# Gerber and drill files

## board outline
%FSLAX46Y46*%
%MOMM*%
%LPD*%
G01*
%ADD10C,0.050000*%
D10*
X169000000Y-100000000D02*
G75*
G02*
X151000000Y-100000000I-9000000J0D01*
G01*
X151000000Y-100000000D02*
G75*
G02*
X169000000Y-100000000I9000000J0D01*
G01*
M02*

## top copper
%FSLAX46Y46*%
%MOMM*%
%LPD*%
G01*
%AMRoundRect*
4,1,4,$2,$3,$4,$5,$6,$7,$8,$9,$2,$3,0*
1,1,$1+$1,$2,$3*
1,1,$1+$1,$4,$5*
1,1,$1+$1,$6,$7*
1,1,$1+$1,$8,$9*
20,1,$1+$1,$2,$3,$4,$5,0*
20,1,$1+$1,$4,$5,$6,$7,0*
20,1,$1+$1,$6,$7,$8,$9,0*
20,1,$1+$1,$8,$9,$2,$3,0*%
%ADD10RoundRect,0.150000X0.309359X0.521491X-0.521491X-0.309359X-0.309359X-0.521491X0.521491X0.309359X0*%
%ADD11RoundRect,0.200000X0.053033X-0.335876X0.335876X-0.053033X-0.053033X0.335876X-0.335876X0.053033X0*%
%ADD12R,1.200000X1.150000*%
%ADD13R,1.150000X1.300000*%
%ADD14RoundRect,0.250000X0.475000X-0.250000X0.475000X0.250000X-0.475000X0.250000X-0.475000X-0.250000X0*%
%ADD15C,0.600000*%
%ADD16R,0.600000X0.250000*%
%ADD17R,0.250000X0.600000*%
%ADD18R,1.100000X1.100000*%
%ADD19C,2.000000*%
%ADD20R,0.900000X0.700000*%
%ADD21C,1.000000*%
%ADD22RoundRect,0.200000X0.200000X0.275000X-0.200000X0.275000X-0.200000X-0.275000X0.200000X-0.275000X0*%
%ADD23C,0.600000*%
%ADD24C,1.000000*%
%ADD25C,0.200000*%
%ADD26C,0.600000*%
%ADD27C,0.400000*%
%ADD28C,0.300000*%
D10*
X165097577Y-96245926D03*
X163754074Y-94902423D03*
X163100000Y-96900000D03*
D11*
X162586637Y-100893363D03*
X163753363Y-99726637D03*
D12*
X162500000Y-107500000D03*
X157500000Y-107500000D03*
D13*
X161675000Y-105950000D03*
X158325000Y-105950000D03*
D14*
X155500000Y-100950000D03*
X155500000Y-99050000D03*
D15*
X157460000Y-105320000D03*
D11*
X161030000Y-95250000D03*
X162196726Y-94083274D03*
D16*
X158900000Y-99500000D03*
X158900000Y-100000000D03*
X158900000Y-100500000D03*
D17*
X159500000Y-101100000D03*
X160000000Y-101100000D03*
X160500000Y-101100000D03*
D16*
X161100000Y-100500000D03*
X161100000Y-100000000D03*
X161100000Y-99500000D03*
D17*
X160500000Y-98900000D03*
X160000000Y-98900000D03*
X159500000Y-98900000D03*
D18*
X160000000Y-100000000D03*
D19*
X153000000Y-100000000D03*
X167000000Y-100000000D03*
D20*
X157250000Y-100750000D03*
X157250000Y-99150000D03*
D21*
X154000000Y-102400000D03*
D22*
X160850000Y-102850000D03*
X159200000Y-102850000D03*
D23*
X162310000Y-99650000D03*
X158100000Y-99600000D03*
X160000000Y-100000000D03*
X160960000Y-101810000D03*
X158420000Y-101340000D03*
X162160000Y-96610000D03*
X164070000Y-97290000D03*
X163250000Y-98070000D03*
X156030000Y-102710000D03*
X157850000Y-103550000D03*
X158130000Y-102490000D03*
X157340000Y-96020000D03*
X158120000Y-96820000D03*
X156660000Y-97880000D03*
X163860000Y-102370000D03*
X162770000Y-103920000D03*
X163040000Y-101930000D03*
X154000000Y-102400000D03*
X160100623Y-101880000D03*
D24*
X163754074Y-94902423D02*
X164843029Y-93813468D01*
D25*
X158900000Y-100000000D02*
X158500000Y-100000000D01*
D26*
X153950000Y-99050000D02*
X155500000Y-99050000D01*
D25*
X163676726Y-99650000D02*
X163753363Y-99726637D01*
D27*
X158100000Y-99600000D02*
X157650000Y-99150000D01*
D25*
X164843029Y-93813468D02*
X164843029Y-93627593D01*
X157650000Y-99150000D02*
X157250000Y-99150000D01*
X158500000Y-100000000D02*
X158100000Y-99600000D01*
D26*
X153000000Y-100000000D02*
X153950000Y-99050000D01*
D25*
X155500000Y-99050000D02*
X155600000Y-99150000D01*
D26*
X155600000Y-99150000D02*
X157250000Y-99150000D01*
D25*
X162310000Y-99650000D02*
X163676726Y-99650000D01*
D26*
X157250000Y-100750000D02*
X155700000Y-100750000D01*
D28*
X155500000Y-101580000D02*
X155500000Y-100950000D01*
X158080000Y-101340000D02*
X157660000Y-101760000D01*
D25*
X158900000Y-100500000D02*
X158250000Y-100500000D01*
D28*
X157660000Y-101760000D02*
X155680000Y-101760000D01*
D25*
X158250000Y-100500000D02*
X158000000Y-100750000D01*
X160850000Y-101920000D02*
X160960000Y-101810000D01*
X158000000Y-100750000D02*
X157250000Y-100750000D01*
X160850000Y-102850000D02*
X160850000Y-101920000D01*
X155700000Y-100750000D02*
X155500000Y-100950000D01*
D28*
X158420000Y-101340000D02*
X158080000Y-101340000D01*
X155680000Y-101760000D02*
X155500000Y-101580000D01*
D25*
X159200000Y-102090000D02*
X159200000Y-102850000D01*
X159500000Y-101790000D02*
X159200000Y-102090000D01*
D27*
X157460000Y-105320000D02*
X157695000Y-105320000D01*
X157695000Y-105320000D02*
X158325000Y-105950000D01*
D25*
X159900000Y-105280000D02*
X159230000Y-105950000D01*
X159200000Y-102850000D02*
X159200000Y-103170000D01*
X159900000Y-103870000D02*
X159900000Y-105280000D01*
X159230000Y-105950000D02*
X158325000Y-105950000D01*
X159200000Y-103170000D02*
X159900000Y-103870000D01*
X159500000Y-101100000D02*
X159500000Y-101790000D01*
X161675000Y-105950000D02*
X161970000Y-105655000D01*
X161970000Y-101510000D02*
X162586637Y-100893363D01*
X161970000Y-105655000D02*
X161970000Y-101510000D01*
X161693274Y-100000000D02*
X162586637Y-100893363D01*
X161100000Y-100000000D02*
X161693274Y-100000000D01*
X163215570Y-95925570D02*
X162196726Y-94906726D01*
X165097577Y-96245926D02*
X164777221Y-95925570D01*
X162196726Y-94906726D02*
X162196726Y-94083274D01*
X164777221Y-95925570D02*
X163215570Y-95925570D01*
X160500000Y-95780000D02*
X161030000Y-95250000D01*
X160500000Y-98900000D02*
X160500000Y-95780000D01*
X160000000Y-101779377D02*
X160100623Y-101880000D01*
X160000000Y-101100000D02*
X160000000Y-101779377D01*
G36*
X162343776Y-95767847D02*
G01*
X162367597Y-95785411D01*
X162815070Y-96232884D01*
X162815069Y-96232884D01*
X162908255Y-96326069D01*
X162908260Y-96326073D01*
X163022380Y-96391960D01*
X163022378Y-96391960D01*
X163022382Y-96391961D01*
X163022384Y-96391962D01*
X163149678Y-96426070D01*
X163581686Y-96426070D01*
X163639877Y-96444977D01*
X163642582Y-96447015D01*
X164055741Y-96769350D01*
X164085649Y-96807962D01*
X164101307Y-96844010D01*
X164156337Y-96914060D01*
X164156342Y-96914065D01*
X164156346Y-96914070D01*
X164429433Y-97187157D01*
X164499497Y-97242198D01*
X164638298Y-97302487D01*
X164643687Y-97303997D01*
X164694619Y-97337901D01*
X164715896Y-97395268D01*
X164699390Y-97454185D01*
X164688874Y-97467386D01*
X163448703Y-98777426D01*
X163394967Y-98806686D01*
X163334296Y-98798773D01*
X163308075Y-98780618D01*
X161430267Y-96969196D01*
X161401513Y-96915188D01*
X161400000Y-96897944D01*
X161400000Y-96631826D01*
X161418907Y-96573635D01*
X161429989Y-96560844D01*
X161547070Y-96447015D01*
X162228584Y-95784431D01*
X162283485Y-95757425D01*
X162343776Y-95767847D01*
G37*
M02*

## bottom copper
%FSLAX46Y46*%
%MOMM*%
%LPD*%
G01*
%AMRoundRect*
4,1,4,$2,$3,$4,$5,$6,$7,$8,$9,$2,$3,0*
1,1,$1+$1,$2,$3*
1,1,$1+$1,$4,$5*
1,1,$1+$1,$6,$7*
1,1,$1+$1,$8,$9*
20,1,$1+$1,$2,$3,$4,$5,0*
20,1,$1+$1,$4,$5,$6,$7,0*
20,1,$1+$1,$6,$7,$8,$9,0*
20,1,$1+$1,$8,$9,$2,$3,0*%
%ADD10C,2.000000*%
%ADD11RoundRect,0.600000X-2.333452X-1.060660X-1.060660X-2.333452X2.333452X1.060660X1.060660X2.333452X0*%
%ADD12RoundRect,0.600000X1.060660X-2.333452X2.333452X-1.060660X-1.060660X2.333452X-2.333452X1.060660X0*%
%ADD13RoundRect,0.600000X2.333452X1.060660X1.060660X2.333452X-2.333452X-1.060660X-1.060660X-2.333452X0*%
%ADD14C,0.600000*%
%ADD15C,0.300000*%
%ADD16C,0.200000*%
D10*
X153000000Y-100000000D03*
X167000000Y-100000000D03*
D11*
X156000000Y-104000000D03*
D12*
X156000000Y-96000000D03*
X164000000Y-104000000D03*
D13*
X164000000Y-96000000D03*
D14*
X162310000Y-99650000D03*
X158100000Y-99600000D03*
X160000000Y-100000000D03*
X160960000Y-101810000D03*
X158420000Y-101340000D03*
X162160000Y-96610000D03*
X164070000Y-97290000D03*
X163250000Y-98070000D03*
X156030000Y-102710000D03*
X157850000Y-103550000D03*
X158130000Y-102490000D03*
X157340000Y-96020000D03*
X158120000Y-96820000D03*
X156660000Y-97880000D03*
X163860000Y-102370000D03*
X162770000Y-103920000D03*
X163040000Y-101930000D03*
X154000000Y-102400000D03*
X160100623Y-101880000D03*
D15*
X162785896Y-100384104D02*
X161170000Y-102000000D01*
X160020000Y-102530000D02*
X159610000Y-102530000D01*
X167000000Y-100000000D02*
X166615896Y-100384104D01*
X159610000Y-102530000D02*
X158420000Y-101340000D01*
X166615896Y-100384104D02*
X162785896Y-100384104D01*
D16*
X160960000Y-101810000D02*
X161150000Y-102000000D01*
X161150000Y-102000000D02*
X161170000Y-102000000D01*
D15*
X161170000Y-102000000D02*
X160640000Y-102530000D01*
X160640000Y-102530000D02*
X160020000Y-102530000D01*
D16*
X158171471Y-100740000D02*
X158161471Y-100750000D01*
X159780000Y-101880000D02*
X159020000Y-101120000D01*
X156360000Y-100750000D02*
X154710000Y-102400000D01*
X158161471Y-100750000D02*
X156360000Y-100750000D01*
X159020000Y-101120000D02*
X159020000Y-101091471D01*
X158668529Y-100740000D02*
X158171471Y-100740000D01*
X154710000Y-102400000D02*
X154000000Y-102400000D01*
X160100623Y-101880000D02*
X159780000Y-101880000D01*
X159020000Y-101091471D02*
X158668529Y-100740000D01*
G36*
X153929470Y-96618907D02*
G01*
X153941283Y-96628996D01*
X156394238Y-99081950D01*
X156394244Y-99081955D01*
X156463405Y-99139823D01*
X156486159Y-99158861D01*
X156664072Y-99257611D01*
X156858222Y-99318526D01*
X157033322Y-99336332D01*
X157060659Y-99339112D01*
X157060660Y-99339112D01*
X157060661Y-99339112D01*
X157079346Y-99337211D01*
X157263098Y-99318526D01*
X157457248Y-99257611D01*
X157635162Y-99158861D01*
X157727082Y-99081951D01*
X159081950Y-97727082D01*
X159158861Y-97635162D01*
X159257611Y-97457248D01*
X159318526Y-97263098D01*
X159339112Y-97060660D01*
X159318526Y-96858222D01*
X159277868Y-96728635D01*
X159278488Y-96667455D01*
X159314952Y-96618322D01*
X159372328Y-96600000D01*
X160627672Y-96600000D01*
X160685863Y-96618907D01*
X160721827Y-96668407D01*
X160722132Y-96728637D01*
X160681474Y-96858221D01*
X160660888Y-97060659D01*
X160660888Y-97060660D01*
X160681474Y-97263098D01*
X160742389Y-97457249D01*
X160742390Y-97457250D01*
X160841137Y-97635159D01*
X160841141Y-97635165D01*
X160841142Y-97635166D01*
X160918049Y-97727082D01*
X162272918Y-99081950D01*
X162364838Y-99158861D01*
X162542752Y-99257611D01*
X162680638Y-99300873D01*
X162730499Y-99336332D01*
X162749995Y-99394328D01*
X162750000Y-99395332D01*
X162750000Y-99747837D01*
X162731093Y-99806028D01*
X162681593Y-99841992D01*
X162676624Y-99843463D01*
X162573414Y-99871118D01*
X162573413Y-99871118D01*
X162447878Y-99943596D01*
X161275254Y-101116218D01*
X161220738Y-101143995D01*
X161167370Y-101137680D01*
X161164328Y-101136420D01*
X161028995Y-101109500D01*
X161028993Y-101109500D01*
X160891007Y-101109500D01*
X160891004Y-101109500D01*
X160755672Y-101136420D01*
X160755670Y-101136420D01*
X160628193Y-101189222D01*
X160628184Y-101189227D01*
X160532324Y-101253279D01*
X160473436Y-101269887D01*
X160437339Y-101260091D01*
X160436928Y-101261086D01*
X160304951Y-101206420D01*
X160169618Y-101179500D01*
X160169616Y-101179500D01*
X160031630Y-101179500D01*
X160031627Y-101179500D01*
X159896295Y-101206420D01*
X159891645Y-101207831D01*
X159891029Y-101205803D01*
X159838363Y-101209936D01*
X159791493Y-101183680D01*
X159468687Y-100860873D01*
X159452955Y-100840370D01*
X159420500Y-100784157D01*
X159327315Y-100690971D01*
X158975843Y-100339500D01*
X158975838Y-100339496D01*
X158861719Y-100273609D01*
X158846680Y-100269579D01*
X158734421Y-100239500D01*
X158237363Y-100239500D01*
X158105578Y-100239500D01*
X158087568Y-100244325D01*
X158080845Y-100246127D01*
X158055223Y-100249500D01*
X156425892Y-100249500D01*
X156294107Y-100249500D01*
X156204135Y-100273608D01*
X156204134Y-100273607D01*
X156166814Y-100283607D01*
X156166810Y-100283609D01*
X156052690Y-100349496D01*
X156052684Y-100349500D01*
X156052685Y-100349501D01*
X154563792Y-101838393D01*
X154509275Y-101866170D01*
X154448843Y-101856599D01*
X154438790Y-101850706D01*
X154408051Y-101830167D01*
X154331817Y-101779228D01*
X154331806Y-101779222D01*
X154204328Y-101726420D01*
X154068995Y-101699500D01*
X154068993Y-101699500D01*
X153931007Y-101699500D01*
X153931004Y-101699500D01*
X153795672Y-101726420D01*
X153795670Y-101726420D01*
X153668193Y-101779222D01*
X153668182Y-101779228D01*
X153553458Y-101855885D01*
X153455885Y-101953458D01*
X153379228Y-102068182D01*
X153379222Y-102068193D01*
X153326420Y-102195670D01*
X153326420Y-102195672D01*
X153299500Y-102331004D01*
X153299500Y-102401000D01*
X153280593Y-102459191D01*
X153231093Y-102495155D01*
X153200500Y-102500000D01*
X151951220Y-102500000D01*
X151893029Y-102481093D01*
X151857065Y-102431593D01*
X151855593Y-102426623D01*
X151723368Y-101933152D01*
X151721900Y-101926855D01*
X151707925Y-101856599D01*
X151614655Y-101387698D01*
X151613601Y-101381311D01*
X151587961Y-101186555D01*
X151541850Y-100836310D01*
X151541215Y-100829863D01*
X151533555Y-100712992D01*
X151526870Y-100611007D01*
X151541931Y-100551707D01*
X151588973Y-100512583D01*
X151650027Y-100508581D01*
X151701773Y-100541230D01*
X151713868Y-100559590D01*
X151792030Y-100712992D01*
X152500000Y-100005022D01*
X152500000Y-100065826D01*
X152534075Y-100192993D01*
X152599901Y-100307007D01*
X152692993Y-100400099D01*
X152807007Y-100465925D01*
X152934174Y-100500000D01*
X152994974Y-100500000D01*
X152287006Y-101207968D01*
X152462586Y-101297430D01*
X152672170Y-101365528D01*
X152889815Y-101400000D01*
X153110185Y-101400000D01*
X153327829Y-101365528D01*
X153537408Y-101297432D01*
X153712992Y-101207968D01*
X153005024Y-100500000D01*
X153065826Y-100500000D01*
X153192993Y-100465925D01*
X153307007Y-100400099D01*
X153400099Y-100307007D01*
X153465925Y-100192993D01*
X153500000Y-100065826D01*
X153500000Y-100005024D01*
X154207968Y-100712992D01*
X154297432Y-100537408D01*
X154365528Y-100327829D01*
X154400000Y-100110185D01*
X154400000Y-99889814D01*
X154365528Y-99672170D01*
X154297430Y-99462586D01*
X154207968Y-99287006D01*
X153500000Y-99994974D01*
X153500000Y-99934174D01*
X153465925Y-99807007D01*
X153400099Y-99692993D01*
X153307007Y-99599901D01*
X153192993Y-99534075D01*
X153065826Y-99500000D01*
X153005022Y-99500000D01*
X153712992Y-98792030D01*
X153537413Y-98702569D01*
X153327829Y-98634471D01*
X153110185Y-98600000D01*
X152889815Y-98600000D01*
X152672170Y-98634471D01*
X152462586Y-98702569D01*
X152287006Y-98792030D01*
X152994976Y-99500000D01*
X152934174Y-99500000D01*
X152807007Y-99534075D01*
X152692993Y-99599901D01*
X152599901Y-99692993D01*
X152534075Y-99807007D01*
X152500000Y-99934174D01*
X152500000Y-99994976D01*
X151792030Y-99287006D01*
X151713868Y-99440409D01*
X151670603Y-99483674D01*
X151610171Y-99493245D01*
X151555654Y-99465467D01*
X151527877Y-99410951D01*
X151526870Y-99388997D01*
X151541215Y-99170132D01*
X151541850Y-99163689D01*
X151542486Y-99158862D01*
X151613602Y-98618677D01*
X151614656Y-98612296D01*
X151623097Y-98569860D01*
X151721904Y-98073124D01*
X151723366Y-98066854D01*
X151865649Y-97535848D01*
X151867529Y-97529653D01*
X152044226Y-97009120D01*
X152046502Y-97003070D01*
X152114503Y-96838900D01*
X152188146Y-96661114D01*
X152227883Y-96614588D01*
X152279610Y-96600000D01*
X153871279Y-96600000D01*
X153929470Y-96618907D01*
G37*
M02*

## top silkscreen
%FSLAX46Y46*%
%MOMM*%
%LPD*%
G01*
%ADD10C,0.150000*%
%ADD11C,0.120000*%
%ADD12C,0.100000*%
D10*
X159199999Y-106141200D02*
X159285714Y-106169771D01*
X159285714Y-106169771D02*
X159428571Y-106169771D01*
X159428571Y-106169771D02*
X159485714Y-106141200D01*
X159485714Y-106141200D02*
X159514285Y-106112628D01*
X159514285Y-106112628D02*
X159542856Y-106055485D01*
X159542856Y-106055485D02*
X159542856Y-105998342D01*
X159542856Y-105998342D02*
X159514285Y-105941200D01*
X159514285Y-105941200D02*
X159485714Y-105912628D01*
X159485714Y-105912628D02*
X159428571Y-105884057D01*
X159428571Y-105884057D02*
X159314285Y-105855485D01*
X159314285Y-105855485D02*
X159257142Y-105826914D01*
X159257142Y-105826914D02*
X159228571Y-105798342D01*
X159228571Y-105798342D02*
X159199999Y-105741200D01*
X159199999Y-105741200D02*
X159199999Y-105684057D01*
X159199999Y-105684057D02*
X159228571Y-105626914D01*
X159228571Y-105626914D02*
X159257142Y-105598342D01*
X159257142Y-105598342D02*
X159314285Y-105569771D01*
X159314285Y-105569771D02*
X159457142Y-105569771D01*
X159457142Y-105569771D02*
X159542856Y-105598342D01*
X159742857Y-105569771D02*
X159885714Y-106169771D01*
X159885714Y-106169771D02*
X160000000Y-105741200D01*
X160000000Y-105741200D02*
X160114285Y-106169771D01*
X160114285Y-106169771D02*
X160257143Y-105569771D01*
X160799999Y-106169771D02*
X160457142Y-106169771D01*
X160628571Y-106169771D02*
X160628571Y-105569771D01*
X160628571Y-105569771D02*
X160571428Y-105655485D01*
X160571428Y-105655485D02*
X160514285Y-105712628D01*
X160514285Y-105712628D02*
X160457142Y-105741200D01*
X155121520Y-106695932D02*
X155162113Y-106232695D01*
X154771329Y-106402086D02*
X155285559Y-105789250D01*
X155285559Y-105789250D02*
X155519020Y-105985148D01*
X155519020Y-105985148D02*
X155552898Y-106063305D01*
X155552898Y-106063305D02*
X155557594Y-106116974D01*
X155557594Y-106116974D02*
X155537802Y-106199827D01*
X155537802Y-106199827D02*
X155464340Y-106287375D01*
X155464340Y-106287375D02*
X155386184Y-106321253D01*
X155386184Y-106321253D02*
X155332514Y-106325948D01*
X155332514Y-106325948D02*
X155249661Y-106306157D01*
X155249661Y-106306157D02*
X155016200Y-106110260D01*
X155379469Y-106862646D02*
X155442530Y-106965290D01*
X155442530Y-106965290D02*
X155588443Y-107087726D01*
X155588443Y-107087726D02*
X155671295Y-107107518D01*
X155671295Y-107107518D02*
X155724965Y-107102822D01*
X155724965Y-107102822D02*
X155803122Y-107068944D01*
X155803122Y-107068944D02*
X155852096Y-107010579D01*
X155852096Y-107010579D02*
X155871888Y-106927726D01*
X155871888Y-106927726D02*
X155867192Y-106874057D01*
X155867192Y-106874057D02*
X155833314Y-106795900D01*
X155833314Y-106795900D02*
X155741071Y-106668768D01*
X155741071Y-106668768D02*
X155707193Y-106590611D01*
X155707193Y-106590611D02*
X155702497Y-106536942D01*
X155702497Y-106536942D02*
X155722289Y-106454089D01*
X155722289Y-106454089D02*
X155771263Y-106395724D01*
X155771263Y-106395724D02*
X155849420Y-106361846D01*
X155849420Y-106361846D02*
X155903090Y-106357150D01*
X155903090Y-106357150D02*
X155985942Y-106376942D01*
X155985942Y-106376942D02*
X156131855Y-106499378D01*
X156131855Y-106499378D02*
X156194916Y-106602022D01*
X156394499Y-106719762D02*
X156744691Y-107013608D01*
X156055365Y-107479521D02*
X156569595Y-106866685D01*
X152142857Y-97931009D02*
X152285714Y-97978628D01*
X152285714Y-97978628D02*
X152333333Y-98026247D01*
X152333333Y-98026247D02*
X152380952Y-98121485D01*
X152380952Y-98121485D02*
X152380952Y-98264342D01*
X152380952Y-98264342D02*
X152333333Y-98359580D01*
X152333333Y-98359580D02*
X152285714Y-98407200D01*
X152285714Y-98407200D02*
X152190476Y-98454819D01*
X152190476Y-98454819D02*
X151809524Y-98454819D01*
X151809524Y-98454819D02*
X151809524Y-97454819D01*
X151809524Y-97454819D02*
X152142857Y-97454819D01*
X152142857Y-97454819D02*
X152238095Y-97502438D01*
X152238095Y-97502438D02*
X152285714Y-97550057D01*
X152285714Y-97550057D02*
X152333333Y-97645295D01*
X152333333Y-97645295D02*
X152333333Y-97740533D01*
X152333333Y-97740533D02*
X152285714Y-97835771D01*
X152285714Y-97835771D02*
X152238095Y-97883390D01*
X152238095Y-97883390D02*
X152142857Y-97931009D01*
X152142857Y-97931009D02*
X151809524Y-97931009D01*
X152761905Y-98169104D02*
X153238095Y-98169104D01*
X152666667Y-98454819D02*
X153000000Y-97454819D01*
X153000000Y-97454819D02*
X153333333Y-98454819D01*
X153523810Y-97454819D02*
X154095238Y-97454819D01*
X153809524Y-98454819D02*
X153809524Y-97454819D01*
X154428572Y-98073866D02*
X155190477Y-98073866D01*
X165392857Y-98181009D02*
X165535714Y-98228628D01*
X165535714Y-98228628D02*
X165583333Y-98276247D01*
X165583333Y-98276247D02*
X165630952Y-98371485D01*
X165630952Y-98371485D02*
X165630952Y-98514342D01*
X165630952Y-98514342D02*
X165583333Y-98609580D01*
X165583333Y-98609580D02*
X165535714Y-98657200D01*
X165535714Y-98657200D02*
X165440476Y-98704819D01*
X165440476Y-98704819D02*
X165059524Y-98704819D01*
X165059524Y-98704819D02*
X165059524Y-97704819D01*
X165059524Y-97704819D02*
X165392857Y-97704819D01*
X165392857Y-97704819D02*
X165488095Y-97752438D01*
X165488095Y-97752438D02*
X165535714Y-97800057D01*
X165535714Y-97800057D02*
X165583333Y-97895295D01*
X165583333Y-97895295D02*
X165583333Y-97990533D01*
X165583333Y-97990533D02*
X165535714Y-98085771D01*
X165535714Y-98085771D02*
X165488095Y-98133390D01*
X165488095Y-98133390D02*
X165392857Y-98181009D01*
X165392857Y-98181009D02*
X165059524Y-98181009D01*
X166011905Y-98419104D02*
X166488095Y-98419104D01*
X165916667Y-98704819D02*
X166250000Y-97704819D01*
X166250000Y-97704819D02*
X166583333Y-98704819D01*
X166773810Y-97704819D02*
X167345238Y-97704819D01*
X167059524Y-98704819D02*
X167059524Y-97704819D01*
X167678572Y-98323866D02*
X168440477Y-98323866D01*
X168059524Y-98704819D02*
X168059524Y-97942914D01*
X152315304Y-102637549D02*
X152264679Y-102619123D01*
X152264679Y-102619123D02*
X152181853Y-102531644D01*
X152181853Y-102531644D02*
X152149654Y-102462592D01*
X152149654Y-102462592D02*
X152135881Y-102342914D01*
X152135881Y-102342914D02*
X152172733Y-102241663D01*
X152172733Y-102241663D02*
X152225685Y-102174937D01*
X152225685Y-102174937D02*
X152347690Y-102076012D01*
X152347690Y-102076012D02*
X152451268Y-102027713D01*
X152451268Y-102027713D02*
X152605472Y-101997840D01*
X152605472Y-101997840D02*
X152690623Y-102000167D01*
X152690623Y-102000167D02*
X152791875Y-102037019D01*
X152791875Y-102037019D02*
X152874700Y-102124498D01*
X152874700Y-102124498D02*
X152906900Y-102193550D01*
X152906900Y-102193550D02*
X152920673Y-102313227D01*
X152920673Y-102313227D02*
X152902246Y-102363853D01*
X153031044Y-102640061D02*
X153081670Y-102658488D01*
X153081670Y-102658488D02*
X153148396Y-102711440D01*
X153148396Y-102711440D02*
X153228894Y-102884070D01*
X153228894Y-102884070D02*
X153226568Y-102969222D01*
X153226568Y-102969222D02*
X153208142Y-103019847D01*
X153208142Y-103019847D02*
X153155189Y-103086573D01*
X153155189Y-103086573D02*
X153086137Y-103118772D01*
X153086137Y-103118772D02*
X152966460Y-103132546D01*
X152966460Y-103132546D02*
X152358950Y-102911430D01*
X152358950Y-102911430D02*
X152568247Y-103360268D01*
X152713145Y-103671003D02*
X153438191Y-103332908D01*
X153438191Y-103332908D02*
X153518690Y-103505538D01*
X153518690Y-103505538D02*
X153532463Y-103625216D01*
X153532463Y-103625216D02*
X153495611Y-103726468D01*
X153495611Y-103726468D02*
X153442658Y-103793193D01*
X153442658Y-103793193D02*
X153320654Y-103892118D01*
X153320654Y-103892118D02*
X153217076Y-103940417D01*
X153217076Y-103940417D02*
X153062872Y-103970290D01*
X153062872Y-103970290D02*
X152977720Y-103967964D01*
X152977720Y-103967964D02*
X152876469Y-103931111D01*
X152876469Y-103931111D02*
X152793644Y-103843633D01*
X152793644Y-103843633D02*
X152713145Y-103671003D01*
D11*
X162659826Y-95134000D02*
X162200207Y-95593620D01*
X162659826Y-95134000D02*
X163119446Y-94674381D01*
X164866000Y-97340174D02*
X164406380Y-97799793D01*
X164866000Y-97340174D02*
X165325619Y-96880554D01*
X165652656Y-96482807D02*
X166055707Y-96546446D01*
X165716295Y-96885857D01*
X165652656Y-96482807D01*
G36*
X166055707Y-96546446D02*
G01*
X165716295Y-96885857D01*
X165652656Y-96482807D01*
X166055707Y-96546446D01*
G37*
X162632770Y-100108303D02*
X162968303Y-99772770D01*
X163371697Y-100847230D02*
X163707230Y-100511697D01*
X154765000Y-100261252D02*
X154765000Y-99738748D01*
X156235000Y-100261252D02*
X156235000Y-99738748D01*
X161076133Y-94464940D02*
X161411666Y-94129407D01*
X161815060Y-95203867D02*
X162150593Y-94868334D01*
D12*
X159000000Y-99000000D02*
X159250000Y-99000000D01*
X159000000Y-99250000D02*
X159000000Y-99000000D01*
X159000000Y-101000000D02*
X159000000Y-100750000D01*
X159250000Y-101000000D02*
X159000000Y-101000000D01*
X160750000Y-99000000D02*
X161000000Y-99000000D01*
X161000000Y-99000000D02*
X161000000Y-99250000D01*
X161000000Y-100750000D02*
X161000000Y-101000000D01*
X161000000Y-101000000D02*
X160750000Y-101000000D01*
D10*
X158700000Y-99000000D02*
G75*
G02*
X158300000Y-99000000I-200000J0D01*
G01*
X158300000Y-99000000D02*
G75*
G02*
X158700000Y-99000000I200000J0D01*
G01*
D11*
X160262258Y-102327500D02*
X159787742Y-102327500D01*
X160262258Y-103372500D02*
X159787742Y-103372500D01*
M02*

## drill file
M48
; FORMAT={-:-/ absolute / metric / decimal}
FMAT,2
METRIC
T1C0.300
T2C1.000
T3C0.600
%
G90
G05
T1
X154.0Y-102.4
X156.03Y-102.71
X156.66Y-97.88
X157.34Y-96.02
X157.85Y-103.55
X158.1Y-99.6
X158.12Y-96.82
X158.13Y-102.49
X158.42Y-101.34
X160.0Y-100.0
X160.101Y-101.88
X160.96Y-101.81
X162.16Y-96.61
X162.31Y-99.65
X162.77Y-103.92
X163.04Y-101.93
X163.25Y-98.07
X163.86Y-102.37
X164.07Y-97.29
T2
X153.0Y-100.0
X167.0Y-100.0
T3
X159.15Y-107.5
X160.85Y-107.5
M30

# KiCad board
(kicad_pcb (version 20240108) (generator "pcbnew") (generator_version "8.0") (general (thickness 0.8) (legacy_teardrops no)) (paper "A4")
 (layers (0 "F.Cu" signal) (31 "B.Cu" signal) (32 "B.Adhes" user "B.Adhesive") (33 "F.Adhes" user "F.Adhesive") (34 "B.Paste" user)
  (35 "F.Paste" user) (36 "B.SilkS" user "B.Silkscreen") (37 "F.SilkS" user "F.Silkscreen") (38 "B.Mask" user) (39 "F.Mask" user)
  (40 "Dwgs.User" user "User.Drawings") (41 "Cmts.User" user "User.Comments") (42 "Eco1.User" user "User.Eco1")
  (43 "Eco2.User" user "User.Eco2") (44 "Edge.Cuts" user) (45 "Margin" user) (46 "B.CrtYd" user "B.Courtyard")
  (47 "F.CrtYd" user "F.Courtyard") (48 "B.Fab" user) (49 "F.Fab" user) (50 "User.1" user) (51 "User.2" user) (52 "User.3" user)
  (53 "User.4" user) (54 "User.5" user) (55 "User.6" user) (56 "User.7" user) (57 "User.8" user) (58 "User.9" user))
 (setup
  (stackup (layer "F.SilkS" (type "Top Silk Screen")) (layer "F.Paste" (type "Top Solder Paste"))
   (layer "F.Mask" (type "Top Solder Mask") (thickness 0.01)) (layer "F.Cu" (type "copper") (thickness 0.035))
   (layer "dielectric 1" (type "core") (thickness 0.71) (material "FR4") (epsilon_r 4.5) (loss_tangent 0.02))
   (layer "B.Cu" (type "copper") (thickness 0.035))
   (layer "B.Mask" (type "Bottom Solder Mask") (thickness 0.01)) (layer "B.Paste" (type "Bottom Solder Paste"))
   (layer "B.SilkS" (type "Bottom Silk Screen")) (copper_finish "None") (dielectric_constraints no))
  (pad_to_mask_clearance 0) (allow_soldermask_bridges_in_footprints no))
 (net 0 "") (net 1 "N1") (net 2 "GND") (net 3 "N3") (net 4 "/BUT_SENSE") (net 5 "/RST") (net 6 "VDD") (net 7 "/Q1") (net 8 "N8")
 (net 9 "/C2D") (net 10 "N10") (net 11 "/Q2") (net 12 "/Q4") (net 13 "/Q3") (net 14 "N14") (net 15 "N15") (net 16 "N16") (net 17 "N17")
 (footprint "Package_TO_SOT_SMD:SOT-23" (layer "F.Cu") (at 163.762913 96.237087 -135)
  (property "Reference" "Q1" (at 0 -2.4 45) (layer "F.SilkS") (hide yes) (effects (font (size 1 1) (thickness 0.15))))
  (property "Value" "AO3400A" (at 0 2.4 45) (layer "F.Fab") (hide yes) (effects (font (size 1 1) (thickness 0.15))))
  (fp_line (start 0 1.560001) (end 0.65 1.56) (stroke (width 0.12) (type solid)) (layer "F.SilkS"))
  (fp_line (start 0 1.560001) (end -0.65 1.56) (stroke (width 0.12) (type solid)) (layer "F.SilkS"))
  (fp_line (start 0 -1.560001) (end 0.65 -1.56) (stroke (width 0.12) (type solid)) (layer "F.SilkS"))
  (fp_line (start 0 -1.560001) (end -0.65 -1.56) (stroke (width 0.12) (type solid)) (layer "F.SilkS"))
  (fp_poly
   (pts (xy -1.1625 -1.51) (xy -1.4025 -1.84) (xy -0.9225 -1.839999) (xy -1.1625 -1.51)) (stroke (width 0.12) (type solid)) (fill solid)
   (layer "F.SilkS"))
  (pad "1" smd roundrect (at -0.9375 -0.95 225) (size 1.475 0.6) (layers "F.Cu" "F.Paste" "F.Mask") (roundrect_rratio 0.25) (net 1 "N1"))
  (pad "2" smd roundrect (at -0.9375 0.95 225) (size 1.475 0.6) (layers "F.Cu" "F.Paste" "F.Mask") (roundrect_rratio 0.25) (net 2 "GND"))
  (pad "3" smd roundrect (at 0.937501 0 225) (size 1.475 0.6) (layers "F.Cu" "F.Paste" "F.Mask") (roundrect_rratio 0.25) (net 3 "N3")))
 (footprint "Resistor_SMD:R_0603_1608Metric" (layer "F.Cu") (at 163.17 100.31 45)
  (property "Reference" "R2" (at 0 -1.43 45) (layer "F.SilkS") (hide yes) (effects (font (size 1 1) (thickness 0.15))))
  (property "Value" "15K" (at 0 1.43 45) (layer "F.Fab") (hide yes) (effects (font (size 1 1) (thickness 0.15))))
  (fp_line (start -0.237258 -0.5225) (end 0.237258 -0.5225) (stroke (width 0.12) (type solid)) (layer "F.SilkS"))
  (fp_line (start -0.237258 0.5225) (end 0.237258 0.5225) (stroke (width 0.12) (type solid)) (layer "F.SilkS"))
  (pad "1" smd roundrect (at -0.825 0 45) (size 0.8 0.95) (layers "F.Cu" "F.Paste" "F.Mask") (roundrect_rratio 0.25) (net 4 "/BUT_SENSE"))
  (pad "2" smd roundrect (at 0.825 0 45) (size 0.8 0.95) (layers "F.Cu" "F.Paste" "F.Mask") (roundrect_rratio 0.25) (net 2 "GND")))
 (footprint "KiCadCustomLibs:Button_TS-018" (layer "F.Cu") (at 160 107.5 180)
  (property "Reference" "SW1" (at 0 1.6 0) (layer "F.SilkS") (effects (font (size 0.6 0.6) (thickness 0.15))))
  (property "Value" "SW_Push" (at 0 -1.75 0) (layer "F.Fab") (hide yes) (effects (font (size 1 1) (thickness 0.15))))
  (pad "" smd rect (at -2.5 0 270) (size 1.15 1.2) (layers "F.Cu" "F.Paste" "F.Mask"))
  (pad "" np_thru_hole circle (at -0.85 0 180) (size 0.6 0.6) (drill 0.6) (layers "*.Cu" "*.Mask"))
  (pad "" np_thru_hole circle (at 0.85 0 180) (size 0.6 0.6) (drill 0.6) (layers "*.Cu" "*.Mask"))
  (pad "" smd rect (at 2.5 0 270) (size 1.15 1.2) (layers "F.Cu" "F.Paste" "F.Mask"))
  (pad "1" smd rect (at -1.675 1.55 180) (size 1.15 1.3) (layers "F.Cu" "F.Paste" "F.Mask") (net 4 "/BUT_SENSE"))
  (pad "2" smd rect (at 1.675 1.55 180) (size 1.15 1.3) (layers "F.Cu" "F.Paste" "F.Mask") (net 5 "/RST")))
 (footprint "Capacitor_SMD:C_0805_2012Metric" (layer "F.Cu") (at 155.5 100 90)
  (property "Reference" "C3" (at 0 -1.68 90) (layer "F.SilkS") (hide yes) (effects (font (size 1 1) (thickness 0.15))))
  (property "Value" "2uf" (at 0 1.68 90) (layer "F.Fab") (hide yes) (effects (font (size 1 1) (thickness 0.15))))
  (fp_line (start -0.261252 -0.735) (end 0.261252 -0.735) (stroke (width 0.12) (type solid)) (layer "F.SilkS"))
  (fp_line (start -0.261252 0.735) (end 0.261252 0.735) (stroke (width 0.12) (type solid)) (layer "F.SilkS"))
  (pad "1" smd roundrect (at -0.95 0 90) (size 1 1.45) (layers "F.Cu" "F.Paste" "F.Mask") (roundrect_rratio 0.25) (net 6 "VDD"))
  (pad "2" smd roundrect (at 0.95 0 90) (size 1 1.45) (layers "F.Cu" "F.Paste" "F.Mask") (roundrect_rratio 0.25) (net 2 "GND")))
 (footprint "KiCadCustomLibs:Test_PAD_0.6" (layer "F.Cu") (at 157.46 105.32)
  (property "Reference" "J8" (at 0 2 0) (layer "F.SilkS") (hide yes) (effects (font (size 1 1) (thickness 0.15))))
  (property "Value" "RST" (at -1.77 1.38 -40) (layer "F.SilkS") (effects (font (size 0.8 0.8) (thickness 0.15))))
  (pad "1" smd circle (at 0 0) (size 0.6 0.6) (layers "F.Cu" "F.Mask") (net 5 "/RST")))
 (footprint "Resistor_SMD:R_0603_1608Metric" (layer "F.Cu") (at 161.613363 94.666637 45)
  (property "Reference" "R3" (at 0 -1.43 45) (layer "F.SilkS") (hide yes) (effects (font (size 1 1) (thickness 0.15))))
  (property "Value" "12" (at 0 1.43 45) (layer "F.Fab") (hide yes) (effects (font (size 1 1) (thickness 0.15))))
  (fp_line (start -0.237258 -0.5225) (end 0.237258 -0.5225) (stroke (width 0.12) (type solid)) (layer "F.SilkS"))
  (fp_line (start -0.237258 0.5225) (end 0.237258 0.5225) (stroke (width 0.12) (type solid)) (layer "F.SilkS"))
  (pad "1" smd roundrect (at -0.825 0 45) (size 0.8 0.95) (layers "F.Cu" "F.Paste" "F.Mask") (roundrect_rratio 0.25) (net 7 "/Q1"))
  (pad "2" smd roundrect (at 0.825 0 45) (size 0.8 0.95) (layers "F.Cu" "F.Paste" "F.Mask") (roundrect_rratio 0.25) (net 1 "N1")))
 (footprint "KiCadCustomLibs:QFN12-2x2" (layer "F.Cu") (at 160 100)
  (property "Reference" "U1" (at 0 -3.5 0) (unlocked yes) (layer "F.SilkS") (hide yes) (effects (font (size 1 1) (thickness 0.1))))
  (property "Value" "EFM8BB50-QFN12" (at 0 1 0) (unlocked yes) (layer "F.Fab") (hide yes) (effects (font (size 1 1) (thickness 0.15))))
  (fp_line (start -1 -1) (end -0.75 -1) (stroke (width 0.1) (type default)) (layer "F.SilkS"))
  (fp_line (start -1 -0.75) (end -1 -1) (stroke (width 0.1) (type default)) (layer "F.SilkS"))
  (fp_line (start -1 1) (end -1 0.75) (stroke (width 0.1) (type default)) (layer "F.SilkS"))
  (fp_line (start -0.75 1) (end -1 1) (stroke (width 0.1) (type default)) (layer "F.SilkS"))
  (fp_line (start 0.75 -1) (end 1 -1) (stroke (width 0.1) (type default)) (layer "F.SilkS"))
  (fp_line (start 1 -1) (end 1 -0.75) (stroke (width 0.1) (type default)) (layer "F.SilkS"))
  (fp_line (start 1 0.75) (end 1 1) (stroke (width 0.1) (type default)) (layer "F.SilkS"))
  (fp_line (start 1 1) (end 0.75 1) (stroke (width 0.1) (type default)) (layer "F.SilkS"))
  (fp_circle (center -1.5 -1) (end -1.3 -1) (stroke (width 0.15) (type default)) (fill none) (layer "F.SilkS"))
  (pad "1" smd rect (at -1.1 -0.5) (size 0.6 0.25) (layers "F.Cu" "F.Paste" "F.Mask") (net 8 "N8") (thermal_bridge_angle 45))
  (pad "2" smd rect (at -1.1 0) (size 0.6 0.25) (layers "F.Cu" "F.Paste" "F.Mask") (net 2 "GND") (thermal_bridge_angle 45))
  (pad "3" smd rect (at -1.1 0.5) (size 0.6 0.25) (layers "F.Cu" "F.Paste" "F.Mask") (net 6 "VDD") (thermal_bridge_angle 45))
  (pad "4" smd rect (at -0.5 1.1) (size 0.25 0.6) (layers "F.Cu" "F.Paste" "F.Mask") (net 5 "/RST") (thermal_bridge_angle 45))
  (pad "5" smd rect (at 0 1.1) (size 0.25 0.6) (layers "F.Cu" "F.Paste" "F.Mask") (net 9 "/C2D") (thermal_bridge_angle 45))
  (pad "6" smd rect (at 0.5 1.1) (size 0.25 0.6) (layers "F.Cu" "F.Paste" "F.Mask") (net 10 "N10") (thermal_bridge_angle 45))
  (pad "7" smd rect (at 1.1 0.5) (size 0.6 0.25) (layers "F.Cu" "F.Paste" "F.Mask") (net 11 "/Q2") (thermal_bridge_angle 45))
  (pad "8" smd rect (at 1.1 0) (size 0.6 0.25) (layers "F.Cu" "F.Paste" "F.Mask") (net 4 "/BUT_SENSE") (thermal_bridge_angle 45))
  (pad "9" smd rect (at 1.1 -0.5) (size 0.6 0.25) (layers "F.Cu" "F.Paste" "F.Mask") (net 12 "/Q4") (thermal_bridge_angle 45))
  (pad "10" smd rect (at 0.5 -1.1) (size 0.25 0.6) (layers "F.Cu" "F.Paste" "F.Mask") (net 7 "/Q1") (thermal_bridge_angle 45))
  (pad "11" smd rect (at 0 -1.1) (size 0.25 0.6) (layers "F.Cu" "F.Paste" "F.Mask") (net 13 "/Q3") (thermal_bridge_angle 45))
  (pad "12" smd rect (at -0.5 -1.1) (size 0.25 0.6) (layers "F.Cu" "F.Paste" "F.Mask") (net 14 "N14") (thermal_bridge_angle 45))
  (pad "13" smd rect (at 0 0) (size 1.1 1.1) (layers "F.Cu" "F.Paste" "F.Mask") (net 2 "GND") (thermal_bridge_angle 45)))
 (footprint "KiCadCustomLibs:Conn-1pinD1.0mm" (layer "F.Cu") (at 153 100)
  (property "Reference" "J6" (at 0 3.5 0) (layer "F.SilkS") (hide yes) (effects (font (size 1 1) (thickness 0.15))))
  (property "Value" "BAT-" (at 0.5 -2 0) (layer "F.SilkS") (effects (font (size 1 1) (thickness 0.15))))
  (pad "1" thru_hole circle (at 0 0) (size 2 2) (drill 1) (layers "*.Cu" "*.Mask") (remove_unused_layers no) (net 2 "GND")))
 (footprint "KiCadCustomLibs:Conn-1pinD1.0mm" (layer "F.Cu") (at 167 100)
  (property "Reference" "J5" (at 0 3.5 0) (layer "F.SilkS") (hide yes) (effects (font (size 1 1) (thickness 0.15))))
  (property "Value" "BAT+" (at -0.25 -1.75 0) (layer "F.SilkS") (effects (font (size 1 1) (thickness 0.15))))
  (pad "1" thru_hole circle (at 0 0) (size 2 2) (drill 1) (layers "*.Cu" "*.Mask") (remove_unused_layers no) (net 6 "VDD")))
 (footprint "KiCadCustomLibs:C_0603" (layer "F.Cu") (at 157.25 99.95 90)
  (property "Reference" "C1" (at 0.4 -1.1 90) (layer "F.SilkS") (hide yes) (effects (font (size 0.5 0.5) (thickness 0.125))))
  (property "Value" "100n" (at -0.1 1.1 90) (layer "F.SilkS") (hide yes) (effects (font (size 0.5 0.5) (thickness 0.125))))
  (pad "1" smd rect (at -0.8 0 90) (size 0.7 0.9) (layers "F.Cu" "F.Paste" "F.Mask") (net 6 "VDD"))
  (pad "2" smd rect (at 0.8 0 90) (size 0.7 0.9) (layers "F.Cu" "F.Paste" "F.Mask") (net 2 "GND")))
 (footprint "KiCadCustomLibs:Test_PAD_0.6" (layer "F.Cu") (at 154 102.4)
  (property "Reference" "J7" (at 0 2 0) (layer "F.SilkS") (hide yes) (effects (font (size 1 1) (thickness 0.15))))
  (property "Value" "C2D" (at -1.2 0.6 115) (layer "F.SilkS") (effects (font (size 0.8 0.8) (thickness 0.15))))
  (pad "1" smd circle (at 0 0) (size 1 1) (layers "F.Cu" "F.Mask") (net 9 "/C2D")))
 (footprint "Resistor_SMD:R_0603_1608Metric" (layer "F.Cu") (at 160.025 102.85 180)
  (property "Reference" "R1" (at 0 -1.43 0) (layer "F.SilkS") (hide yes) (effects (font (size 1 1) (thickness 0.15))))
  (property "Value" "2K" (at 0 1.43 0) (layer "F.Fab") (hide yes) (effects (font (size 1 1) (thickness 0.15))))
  (fp_line (start -0.237258 0.5225) (end 0.237258 0.5225) (stroke (width 0.12) (type solid)) (layer "F.SilkS"))
  (fp_line (start -0.237258 -0.5225) (end 0.237258 -0.5225) (stroke (width 0.12) (type solid)) (layer "F.SilkS"))
  (pad "1" smd roundrect (at -0.825 0 180) (size 0.8 0.95) (layers "F.Cu" "F.Paste" "F.Mask") (roundrect_rratio 0.25) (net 6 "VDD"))
  (pad "2" smd roundrect (at 0.825 0 180) (size 0.8 0.95) (layers "F.Cu" "F.Paste" "F.Mask") (roundrect_rratio 0.25) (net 5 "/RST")))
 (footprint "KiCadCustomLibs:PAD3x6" (layer "B.Cu") (at 156 104 -45)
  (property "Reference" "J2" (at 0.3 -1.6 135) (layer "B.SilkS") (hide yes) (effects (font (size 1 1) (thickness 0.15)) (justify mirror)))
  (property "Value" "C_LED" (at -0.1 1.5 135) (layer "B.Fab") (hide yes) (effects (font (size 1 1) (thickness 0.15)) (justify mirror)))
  (pad "1" smd roundrect (at 0 0 315) (size 3 6) (layers "B.Cu" "B.Paste" "B.Mask") (roundrect_rratio 0.2) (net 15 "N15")))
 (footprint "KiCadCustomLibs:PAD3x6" (layer "B.Cu") (at 156 96 45)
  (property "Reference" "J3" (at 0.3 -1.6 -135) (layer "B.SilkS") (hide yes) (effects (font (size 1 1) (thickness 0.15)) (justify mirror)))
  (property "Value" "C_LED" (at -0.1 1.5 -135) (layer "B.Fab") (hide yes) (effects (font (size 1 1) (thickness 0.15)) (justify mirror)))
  (pad "1" smd roundrect (at 0 0 45) (size 3 6) (layers "B.Cu" "B.Paste" "B.Mask") (roundrect_rratio 0.2) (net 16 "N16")))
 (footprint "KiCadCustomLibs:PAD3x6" (layer "B.Cu") (at 164 104 45)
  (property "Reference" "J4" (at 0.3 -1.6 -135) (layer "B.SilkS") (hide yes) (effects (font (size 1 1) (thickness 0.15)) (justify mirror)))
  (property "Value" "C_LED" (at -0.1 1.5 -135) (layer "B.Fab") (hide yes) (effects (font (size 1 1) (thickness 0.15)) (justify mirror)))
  (pad "1" smd roundrect (at 0 0 45) (size 3 6) (layers "B.Cu" "B.Paste" "B.Mask") (roundrect_rratio 0.2) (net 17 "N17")))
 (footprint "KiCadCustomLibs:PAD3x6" (layer "B.Cu") (at 164 96 135)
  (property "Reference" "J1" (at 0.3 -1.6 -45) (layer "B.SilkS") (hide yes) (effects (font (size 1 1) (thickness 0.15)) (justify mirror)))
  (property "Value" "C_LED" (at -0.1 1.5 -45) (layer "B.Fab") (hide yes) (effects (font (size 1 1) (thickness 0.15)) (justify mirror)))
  (pad "1" smd roundrect (at 0 0 135) (size 3 6) (layers "B.Cu" "B.Paste" "B.Mask") (roundrect_rratio 0.2) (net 3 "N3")))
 (gr_circle (center 160 100) (end 160 91) (stroke (width 0.05) (type default)) (fill none) (layer "Edge.Cuts"))
 (segment (start 163.754074 94.902423) (end 164.843029 93.813468) (width 1) (layer "F.Cu") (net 2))
 (segment (start 158.9 100) (end 158.5 100) (width 0.2) (layer "F.Cu") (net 2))
 (segment (start 153.95 99.05) (end 155.5 99.05) (width 0.6) (layer "F.Cu") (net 2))
 (segment (start 163.676726 99.65) (end 163.753363 99.726637) (width 0.2) (layer "F.Cu") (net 2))
 (segment (start 158.1 99.6) (end 157.65 99.15) (width 0.4) (layer "F.Cu") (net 2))
 (segment (start 164.843029 93.813468) (end 164.843029 93.627593) (width 0.2) (layer "F.Cu") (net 2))
 (segment (start 157.65 99.15) (end 157.25 99.15) (width 0.2) (layer "F.Cu") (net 2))
 (segment (start 158.5 100) (end 158.1 99.6) (width 0.2) (layer "F.Cu") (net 2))
 (segment (start 153 100) (end 153.95 99.05) (width 0.6) (layer "F.Cu") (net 2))
 (segment (start 155.5 99.05) (end 155.6 99.15) (width 0.2) (layer "F.Cu") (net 2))
 (segment (start 155.6 99.15) (end 157.25 99.15) (width 0.6) (layer "F.Cu") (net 2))
 (segment (start 162.31 99.65) (end 163.676726 99.65) (width 0.2) (layer "F.Cu") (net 2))
 (via (at 162.31 99.65) (size 0.6) (drill 0.3) (layers "F.Cu" "B.Cu") (free yes) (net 2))
 (via (at 158.1 99.6) (size 0.6) (drill 0.3) (layers "F.Cu" "B.Cu") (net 2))
 (via (at 160 100) (size 0.6) (drill 0.3) (layers "F.Cu" "B.Cu") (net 2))
 (segment (start 157.25 100.75) (end 155.7 100.75) (width 0.6) (layer "F.Cu") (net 6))
 (segment (start 155.5 101.58) (end 155.5 100.95) (width 0.3) (layer "F.Cu") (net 6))
 (segment (start 158.08 101.34) (end 157.66 101.76) (width 0.3) (layer "F.Cu") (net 6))
 (segment (start 158.9 100.5) (end 158.25 100.5) (width 0.2) (layer "F.Cu") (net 6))
 (segment (start 157.66 101.76) (end 155.68 101.76) (width 0.3) (layer "F.Cu") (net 6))
 (segment (start 158.25 100.5) (end 158 100.75) (width 0.2) (layer "F.Cu") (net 6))
 (segment (start 160.85 101.92) (end 160.96 101.81) (width 0.2) (layer "F.Cu") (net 6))
 (segment (start 158 100.75) (end 157.25 100.75) (width 0.2) (layer "F.Cu") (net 6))
 (segment (start 160.85 102.85) (end 160.85 101.92) (width 0.2) (layer "F.Cu") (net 6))
 (segment (start 155.7 100.75) (end 155.5 100.95) (width 0.2) (layer "F.Cu") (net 6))
 (segment (start 158.42 101.34) (end 158.08 101.34) (width 0.3) (layer "F.Cu") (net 6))
 (segment (start 155.68 101.76) (end 155.5 101.58) (width 0.3) (layer "F.Cu") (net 6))
 (via (at 160.96 101.81) (size 0.6) (drill 0.3) (layers "F.Cu" "B.Cu") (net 6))
 (via (at 158.42 101.34) (size 0.6) (drill 0.3) (layers "F.Cu" "B.Cu") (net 6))
 (segment (start 162.785896 100.384104) (end 161.17 102) (width 0.3) (layer "B.Cu") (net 6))
 (segment (start 160.02 102.53) (end 159.61 102.53) (width 0.3) (layer "B.Cu") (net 6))
 (segment (start 167 100) (end 166.615896 100.384104) (width 0.3) (layer "B.Cu") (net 6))
 (segment (start 159.61 102.53) (end 158.42 101.34) (width 0.3) (layer "B.Cu") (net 6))
 (segment (start 166.615896 100.384104) (end 162.785896 100.384104) (width 0.3) (layer "B.Cu") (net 6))
 (segment (start 160.96 101.81) (end 161.15 102) (width 0.2) (layer "B.Cu") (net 6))
 (segment (start 161.15 102) (end 161.17 102) (width 0.2) (layer "B.Cu") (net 6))
 (segment (start 161.17 102) (end 160.64 102.53) (width 0.3) (layer "B.Cu") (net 6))
 (segment (start 160.64 102.53) (end 160.02 102.53) (width 0.3) (layer "B.Cu") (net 6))
 (segment (start 159.2 102.09) (end 159.2 102.85) (width 0.2) (layer "F.Cu") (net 5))
 (segment (start 159.5 101.79) (end 159.2 102.09) (width 0.2) (layer "F.Cu") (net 5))
 (segment (start 157.46 105.32) (end 157.695 105.32) (width 0.4) (layer "F.Cu") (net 5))
 (segment (start 157.695 105.32) (end 158.325 105.95) (width 0.4) (layer "F.Cu") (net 5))
 (segment (start 159.9 105.28) (end 159.23 105.95) (width 0.2) (layer "F.Cu") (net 5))
 (segment (start 159.2 102.85) (end 159.2 103.17) (width 0.2) (layer "F.Cu") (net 5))
 (segment (start 159.9 103.87) (end 159.9 105.28) (width 0.2) (layer "F.Cu") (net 5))
 (segment (start 159.23 105.95) (end 158.325 105.95) (width 0.2) (layer "F.Cu") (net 5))
 (segment (start 159.2 103.17) (end 159.9 103.87) (width 0.2) (layer "F.Cu") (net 5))
 (segment (start 159.5 101.1) (end 159.5 101.79) (width 0.2) (layer "F.Cu") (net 5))
 (segment (start 161.675 105.95) (end 161.97 105.655) (width 0.2) (layer "F.Cu") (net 4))
 (segment (start 161.97 101.51) (end 162.586637 100.893363) (width 0.2) (layer "F.Cu") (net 4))
 (segment (start 161.97 105.655) (end 161.97 101.51) (width 0.2) (layer "F.Cu") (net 4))
 (segment (start 161.693274 100) (end 162.586637 100.893363) (width 0.2) (layer "F.Cu") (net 4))
 (segment (start 161.1 100) (end 161.693274 100) (width 0.2) (layer "F.Cu") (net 4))
 (via (at 162.16 96.61) (size 0.6) (drill 0.3) (layers "F.Cu" "B.Cu") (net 3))
 (via (at 164.07 97.29) (size 0.6) (drill 0.3) (layers "F.Cu" "B.Cu") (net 3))
 (via (at 163.25 98.07) (size 0.6) (drill 0.3) (layers "F.Cu" "B.Cu") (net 3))
 (segment (start 163.21557 95.92557) (end 162.196726 94.906726) (width 0.2) (layer "F.Cu") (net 1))
 (segment (start 165.097577 96.245926) (end 164.777221 95.92557) (width 0.2) (layer "F.Cu") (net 1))
 (segment (start 162.196726 94.906726) (end 162.196726 94.083274) (width 0.2) (layer "F.Cu") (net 1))
 (segment (start 164.777221 95.92557) (end 163.21557 95.92557) (width 0.2) (layer "F.Cu") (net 1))
 (via (at 156.03 102.71) (size 0.6) (drill 0.3) (layers "F.Cu" "B.Cu") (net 15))
 (via (at 157.85 103.55) (size 0.6) (drill 0.3) (layers "F.Cu" "B.Cu") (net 15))
 (via (at 158.13 102.49) (size 0.6) (drill 0.3) (layers "F.Cu" "B.Cu") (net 15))
 (via (at 157.34 96.02) (size 0.6) (drill 0.3) (layers "F.Cu" "B.Cu") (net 16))
 (via (at 158.12 96.82) (size 0.6) (drill 0.3) (layers "F.Cu" "B.Cu") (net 16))
 (via (at 156.66 97.88) (size 0.6) (drill 0.3) (layers "F.Cu" "B.Cu") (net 16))
 (via (at 163.86 102.37) (size 0.6) (drill 0.3) (layers "F.Cu" "B.Cu") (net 17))
 (via (at 162.77 103.92) (size 0.6) (drill 0.3) (layers "F.Cu" "B.Cu") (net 17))
 (via (at 163.04 101.93) (size 0.6) (drill 0.3) (layers "F.Cu" "B.Cu") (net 17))
 (segment (start 160.5 95.78) (end 161.03 95.25) (width 0.2) (layer "F.Cu") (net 7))
 (segment (start 160.5 98.9) (end 160.5 95.78) (width 0.2) (layer "F.Cu") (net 7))
 (segment (start 160 101.779377) (end 160.100623 101.88) (width 0.2) (layer "F.Cu") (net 9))
 (segment (start 160 101.1) (end 160 101.779377) (width 0.2) (layer "F.Cu") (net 9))
 (via (at 154 102.4) (size 0.6) (drill 0.3) (layers "F.Cu" "B.Cu") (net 9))
 (via (at 160.100623 101.88) (size 0.6) (drill 0.3) (layers "F.Cu" "B.Cu") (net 9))
 (segment (start 158.171471 100.74) (end 158.161471 100.75) (width 0.2) (layer "B.Cu") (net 9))
 (segment (start 159.78 101.88) (end 159.02 101.12) (width 0.2) (layer "B.Cu") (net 9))
 (segment (start 156.36 100.75) (end 154.71 102.4) (width 0.2) (layer "B.Cu") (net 9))
 (segment (start 158.161471 100.75) (end 156.36 100.75) (width 0.2) (layer "B.Cu") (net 9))
 (segment (start 159.02 101.12) (end 159.02 101.091471) (width 0.2) (layer "B.Cu") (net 9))
 (segment (start 158.668529 100.74) (end 158.171471 100.74) (width 0.2) (layer "B.Cu") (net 9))
 (segment (start 154.71 102.4) (end 154 102.4) (width 0.2) (layer "B.Cu") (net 9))
 (segment (start 160.100623 101.88) (end 159.78 101.88) (width 0.2) (layer "B.Cu") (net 9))
 (segment (start 159.02 101.091471) (end 158.668529 100.74) (width 0.2) (layer "B.Cu") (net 9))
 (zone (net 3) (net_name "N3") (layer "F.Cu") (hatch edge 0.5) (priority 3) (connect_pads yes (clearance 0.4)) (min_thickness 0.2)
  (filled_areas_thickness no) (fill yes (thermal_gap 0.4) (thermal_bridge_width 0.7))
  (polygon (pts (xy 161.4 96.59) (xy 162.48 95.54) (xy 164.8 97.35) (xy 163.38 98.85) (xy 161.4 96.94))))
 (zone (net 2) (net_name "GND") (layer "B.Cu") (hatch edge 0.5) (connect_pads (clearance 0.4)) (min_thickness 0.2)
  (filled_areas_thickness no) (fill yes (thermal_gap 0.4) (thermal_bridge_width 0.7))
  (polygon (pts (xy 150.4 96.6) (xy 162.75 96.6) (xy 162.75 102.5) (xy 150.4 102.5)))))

